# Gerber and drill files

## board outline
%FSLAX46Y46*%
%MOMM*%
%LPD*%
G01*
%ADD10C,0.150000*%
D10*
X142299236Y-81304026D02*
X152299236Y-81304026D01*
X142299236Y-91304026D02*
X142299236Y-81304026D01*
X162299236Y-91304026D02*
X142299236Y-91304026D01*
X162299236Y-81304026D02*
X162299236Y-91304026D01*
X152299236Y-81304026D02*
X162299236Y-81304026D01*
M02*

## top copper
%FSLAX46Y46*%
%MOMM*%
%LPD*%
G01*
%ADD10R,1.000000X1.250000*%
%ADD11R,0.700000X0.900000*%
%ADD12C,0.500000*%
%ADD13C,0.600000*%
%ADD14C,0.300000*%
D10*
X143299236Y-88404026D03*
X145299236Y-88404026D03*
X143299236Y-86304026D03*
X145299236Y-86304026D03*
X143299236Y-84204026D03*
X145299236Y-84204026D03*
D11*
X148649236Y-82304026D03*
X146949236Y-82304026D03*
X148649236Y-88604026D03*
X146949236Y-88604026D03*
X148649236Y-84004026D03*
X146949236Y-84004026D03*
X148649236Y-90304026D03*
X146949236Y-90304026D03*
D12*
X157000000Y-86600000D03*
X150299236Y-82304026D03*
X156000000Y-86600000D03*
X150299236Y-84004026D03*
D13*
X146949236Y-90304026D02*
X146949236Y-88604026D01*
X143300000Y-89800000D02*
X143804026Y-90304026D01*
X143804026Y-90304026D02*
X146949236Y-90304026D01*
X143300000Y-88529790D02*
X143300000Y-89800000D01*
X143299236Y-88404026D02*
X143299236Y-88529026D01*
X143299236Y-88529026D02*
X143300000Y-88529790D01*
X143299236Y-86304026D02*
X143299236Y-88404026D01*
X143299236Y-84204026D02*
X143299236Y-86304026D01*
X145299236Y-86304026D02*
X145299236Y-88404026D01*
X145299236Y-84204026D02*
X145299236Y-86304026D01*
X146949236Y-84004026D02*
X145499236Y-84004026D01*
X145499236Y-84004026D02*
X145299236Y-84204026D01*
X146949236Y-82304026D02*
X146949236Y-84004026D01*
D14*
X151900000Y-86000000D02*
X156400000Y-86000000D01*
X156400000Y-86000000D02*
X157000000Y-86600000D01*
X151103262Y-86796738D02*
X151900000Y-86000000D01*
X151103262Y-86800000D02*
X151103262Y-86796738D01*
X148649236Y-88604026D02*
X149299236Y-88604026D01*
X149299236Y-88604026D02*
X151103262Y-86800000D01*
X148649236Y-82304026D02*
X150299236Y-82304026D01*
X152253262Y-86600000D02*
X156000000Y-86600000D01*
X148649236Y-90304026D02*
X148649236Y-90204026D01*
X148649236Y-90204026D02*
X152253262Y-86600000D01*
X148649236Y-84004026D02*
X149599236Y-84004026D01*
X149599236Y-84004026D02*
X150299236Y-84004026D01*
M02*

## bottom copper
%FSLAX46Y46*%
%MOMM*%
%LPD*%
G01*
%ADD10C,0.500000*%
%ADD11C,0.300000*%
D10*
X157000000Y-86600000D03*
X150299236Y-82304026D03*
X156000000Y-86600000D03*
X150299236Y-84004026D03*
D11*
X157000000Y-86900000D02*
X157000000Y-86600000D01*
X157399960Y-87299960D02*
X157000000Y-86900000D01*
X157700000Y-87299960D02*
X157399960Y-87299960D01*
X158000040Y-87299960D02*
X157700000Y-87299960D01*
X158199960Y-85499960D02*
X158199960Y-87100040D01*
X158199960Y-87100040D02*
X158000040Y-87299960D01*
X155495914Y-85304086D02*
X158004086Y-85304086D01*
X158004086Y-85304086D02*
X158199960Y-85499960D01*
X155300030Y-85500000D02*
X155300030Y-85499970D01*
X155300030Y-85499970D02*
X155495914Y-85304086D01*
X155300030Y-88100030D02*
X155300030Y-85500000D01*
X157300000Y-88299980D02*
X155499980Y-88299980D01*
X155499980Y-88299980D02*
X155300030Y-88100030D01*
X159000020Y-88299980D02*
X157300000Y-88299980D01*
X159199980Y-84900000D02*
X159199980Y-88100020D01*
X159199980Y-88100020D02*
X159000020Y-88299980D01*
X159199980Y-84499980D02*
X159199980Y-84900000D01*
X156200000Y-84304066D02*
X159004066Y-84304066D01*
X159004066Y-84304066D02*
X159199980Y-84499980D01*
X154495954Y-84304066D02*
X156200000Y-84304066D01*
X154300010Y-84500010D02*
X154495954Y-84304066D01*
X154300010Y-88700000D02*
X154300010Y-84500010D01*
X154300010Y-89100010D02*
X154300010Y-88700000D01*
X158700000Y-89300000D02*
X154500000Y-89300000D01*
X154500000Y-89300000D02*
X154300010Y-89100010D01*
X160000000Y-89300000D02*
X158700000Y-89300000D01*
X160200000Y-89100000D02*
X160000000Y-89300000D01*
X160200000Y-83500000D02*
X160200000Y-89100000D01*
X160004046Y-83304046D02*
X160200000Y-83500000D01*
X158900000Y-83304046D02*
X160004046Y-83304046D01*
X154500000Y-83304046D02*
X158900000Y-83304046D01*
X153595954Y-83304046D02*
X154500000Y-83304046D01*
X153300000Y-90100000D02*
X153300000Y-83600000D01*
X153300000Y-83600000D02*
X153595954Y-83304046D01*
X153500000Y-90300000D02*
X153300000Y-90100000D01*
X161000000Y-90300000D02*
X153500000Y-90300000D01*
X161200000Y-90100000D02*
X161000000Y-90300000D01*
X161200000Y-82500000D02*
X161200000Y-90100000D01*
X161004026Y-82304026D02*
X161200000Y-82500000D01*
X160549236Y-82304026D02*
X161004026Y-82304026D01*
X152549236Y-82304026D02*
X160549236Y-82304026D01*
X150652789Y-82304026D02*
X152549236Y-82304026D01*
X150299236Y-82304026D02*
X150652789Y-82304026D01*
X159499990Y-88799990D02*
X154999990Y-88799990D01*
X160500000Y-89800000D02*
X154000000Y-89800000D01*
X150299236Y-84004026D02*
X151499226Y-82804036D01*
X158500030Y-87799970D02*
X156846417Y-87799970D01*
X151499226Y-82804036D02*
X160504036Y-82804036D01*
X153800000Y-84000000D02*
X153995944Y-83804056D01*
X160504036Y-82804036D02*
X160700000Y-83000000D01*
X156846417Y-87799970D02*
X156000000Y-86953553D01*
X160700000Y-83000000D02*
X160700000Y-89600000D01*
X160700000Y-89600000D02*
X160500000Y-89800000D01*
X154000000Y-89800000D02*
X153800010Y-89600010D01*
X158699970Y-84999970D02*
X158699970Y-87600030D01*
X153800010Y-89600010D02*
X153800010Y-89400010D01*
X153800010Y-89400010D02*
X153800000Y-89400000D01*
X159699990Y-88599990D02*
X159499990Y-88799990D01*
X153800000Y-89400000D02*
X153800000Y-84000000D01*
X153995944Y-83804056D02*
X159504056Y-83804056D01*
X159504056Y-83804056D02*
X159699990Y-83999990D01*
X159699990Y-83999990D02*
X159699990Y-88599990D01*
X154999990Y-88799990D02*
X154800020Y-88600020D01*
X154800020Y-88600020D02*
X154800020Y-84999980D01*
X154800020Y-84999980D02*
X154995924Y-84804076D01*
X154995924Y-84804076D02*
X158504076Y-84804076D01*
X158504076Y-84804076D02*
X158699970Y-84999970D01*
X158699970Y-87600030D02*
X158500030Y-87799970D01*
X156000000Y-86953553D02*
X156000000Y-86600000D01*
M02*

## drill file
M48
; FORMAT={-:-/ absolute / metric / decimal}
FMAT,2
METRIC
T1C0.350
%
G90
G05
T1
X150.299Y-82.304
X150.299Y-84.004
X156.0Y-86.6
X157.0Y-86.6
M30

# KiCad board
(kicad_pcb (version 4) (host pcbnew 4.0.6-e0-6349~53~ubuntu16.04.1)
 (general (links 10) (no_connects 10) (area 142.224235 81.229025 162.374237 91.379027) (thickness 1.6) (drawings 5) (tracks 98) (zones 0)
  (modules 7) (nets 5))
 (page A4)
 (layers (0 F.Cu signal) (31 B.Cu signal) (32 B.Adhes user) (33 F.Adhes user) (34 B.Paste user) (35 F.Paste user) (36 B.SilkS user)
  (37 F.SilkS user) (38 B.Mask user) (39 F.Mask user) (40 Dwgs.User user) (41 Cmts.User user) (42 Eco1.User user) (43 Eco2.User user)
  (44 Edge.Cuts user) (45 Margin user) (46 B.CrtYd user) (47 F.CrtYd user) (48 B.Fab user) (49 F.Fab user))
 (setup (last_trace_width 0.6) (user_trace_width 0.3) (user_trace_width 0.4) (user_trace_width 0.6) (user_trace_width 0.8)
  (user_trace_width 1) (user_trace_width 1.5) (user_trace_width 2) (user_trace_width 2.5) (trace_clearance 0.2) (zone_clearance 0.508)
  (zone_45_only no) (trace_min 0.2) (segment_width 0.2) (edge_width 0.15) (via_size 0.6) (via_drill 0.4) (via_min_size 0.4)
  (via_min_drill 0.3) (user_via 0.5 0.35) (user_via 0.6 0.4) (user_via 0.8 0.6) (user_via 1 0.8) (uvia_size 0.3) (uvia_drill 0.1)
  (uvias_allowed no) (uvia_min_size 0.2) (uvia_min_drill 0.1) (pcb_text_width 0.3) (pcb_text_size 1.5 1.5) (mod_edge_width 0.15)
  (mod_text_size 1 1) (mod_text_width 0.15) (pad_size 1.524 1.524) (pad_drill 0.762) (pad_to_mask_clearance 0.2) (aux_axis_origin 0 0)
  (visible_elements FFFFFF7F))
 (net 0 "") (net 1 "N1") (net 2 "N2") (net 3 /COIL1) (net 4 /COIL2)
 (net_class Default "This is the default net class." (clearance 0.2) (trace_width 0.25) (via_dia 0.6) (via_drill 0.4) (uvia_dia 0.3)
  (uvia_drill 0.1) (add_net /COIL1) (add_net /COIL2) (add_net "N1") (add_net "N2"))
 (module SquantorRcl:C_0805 (layer F.Cu) (at 144.299236 88.404026)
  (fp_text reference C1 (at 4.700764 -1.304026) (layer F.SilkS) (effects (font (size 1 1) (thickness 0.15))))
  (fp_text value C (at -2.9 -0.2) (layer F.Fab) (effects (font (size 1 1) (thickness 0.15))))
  (pad 1 smd rect (at -1 0) (size 1 1.25) (layers F.Cu F.Paste F.Mask) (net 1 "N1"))
  (pad 2 smd rect (at 1 0) (size 1 1.25) (layers F.Cu F.Paste F.Mask) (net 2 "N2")))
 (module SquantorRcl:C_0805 (layer F.Cu) (at 144.299236 86.304026)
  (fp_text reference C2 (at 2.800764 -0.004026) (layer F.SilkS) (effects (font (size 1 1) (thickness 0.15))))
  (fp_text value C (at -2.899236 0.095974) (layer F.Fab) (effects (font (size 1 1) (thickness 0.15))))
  (pad 1 smd rect (at -1 0) (size 1 1.25) (layers F.Cu F.Paste F.Mask) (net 1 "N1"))
  (pad 2 smd rect (at 1 0) (size 1 1.25) (layers F.Cu F.Paste F.Mask) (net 2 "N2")))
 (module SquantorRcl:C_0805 (layer F.Cu) (at 144.299236 84.204026)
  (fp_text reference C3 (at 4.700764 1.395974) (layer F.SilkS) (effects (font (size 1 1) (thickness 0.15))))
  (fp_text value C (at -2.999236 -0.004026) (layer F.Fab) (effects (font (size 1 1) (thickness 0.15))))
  (pad 1 smd rect (at -1 0) (size 1 1.25) (layers F.Cu F.Paste F.Mask) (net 1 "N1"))
  (pad 2 smd rect (at 1 0) (size 1 1.25) (layers F.Cu F.Paste F.Mask) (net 2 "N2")))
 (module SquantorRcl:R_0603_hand (layer F.Cu) (at 147.799236 82.304026 180)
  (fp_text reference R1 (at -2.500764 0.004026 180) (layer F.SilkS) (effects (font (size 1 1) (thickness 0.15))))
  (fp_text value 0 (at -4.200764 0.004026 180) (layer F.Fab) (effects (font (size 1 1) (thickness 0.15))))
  (pad 1 smd rect (at -0.85 0 180) (size 0.7 0.9) (layers F.Cu F.Paste F.Mask) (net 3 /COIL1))
  (pad 2 smd rect (at 0.85 0 180) (size 0.7 0.9) (layers F.Cu F.Paste F.Mask) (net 2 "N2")))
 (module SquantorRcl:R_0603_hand (layer F.Cu) (at 147.799236 88.604026 180)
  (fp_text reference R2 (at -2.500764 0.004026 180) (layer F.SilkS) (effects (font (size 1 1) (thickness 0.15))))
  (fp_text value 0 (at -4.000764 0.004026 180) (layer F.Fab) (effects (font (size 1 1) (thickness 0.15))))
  (pad 1 smd rect (at -0.85 0 180) (size 0.7 0.9) (layers F.Cu F.Paste F.Mask) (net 3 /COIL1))
  (pad 2 smd rect (at 0.85 0 180) (size 0.7 0.9) (layers F.Cu F.Paste F.Mask) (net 1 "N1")))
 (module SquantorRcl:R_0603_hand (layer F.Cu) (at 147.799236 84.004026 180)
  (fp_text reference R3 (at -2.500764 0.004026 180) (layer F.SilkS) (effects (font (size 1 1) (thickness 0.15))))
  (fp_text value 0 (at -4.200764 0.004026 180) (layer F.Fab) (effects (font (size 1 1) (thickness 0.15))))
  (pad 1 smd rect (at -0.85 0 180) (size 0.7 0.9) (layers F.Cu F.Paste F.Mask) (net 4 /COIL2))
  (pad 2 smd rect (at 0.85 0 180) (size 0.7 0.9) (layers F.Cu F.Paste F.Mask) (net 2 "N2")))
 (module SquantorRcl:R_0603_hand (layer F.Cu) (at 147.799236 90.304026 180)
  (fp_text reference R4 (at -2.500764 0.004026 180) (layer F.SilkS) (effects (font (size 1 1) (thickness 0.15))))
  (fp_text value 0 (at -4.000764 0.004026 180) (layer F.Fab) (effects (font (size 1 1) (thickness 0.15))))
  (pad 1 smd rect (at -0.85 0 180) (size 0.7 0.9) (layers F.Cu F.Paste F.Mask) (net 4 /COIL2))
  (pad 2 smd rect (at 0.85 0 180) (size 0.7 0.9) (layers F.Cu F.Paste F.Mask) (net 1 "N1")))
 (gr_line (start 142.299236 81.304026) (end 152.299236 81.304026) (layer Edge.Cuts) (width 0.15))
 (gr_line (start 142.299236 91.304026) (end 142.299236 81.304026) (layer Edge.Cuts) (width 0.15))
 (gr_line (start 162.299236 91.304026) (end 142.299236 91.304026) (layer Edge.Cuts) (width 0.15))
 (gr_line (start 162.299236 81.304026) (end 162.299236 91.304026) (layer Edge.Cuts) (width 0.15))
 (gr_line (start 152.299236 81.304026) (end 162.299236 81.304026) (layer Edge.Cuts) (width 0.15))
 (segment (start 146.949236 90.304026) (end 146.949236 88.604026) (width 0.6) (layer F.Cu) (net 1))
 (segment (start 143.3 89.8) (end 143.804026 90.304026) (width 0.6) (layer F.Cu) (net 1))
 (segment (start 143.804026 90.304026) (end 146.949236 90.304026) (width 0.6) (layer F.Cu) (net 1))
 (segment (start 143.3 88.52979) (end 143.3 89.8) (width 0.6) (layer F.Cu) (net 1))
 (segment (start 143.299236 88.404026) (end 143.299236 88.529026) (width 0.6) (layer F.Cu) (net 1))
 (segment (start 143.299236 88.529026) (end 143.3 88.52979) (width 0.6) (layer F.Cu) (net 1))
 (segment (start 143.299236 86.304026) (end 143.299236 88.404026) (width 0.6) (layer F.Cu) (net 1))
 (segment (start 143.299236 84.204026) (end 143.299236 86.304026) (width 0.6) (layer F.Cu) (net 1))
 (segment (start 145.299236 86.304026) (end 145.299236 88.404026) (width 0.6) (layer F.Cu) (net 2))
 (segment (start 145.299236 84.204026) (end 145.299236 86.304026) (width 0.6) (layer F.Cu) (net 2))
 (segment (start 146.949236 84.004026) (end 145.499236 84.004026) (width 0.6) (layer F.Cu) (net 2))
 (segment (start 145.499236 84.004026) (end 145.299236 84.204026) (width 0.6) (layer F.Cu) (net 2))
 (segment (start 146.949236 82.304026) (end 146.949236 84.004026) (width 0.6) (layer F.Cu) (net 2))
 (segment (start 151.9 86) (end 156.4 86) (width 0.3) (layer F.Cu) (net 3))
 (segment (start 156.4 86) (end 157 86.6) (width 0.3) (layer F.Cu) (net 3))
 (segment (start 151.103262 86.796738) (end 151.9 86) (width 0.3) (layer F.Cu) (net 3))
 (segment (start 151.103262 86.8) (end 151.103262 86.796738) (width 0.3) (layer F.Cu) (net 3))
 (via (at 157 86.6) (size 0.5) (drill 0.35) (layers F.Cu B.Cu) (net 3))
 (segment (start 157 86.9) (end 157 86.6) (width 0.3) (layer B.Cu) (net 3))
 (segment (start 157.39996 87.29996) (end 157 86.9) (width 0.3) (layer B.Cu) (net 3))
 (segment (start 157.7 87.29996) (end 157.39996 87.29996) (width 0.3) (layer B.Cu) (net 3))
 (segment (start 148.649236 88.604026) (end 149.299236 88.604026) (width 0.3) (layer F.Cu) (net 3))
 (segment (start 149.299236 88.604026) (end 151.103262 86.8) (width 0.3) (layer F.Cu) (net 3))
 (segment (start 158.00004 87.29996) (end 157.7 87.29996) (width 0.3) (layer B.Cu) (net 3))
 (segment (start 158.19996 85.49996) (end 158.19996 87.10004) (width 0.3) (layer B.Cu) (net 3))
 (segment (start 158.19996 87.10004) (end 158.00004 87.29996) (width 0.3) (layer B.Cu) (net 3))
 (segment (start 155.495914 85.304086) (end 158.004086 85.304086) (width 0.3) (layer B.Cu) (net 3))
 (segment (start 158.004086 85.304086) (end 158.19996 85.49996) (width 0.3) (layer B.Cu) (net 3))
 (segment (start 155.30003 85.5) (end 155.30003 85.49997) (width 0.3) (layer B.Cu) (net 3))
 (segment (start 155.30003 85.49997) (end 155.495914 85.304086) (width 0.3) (layer B.Cu) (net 3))
 (segment (start 155.30003 88.10003) (end 155.30003 85.5) (width 0.3) (layer B.Cu) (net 3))
 (segment (start 157.3 88.29998) (end 155.49998 88.29998) (width 0.3) (layer B.Cu) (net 3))
 (segment (start 155.49998 88.29998) (end 155.30003 88.10003) (width 0.3) (layer B.Cu) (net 3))
 (segment (start 159.00002 88.29998) (end 157.3 88.29998) (width 0.3) (layer B.Cu) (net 3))
 (segment (start 159.19998 84.9) (end 159.19998 88.10002) (width 0.3) (layer B.Cu) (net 3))
 (segment (start 159.19998 88.10002) (end 159.00002 88.29998) (width 0.3) (layer B.Cu) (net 3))
 (segment (start 159.19998 84.49998) (end 159.19998 84.9) (width 0.3) (layer B.Cu) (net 3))
 (segment (start 156.2 84.304066) (end 159.004066 84.304066) (width 0.3) (layer B.Cu) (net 3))
 (segment (start 159.004066 84.304066) (end 159.19998 84.49998) (width 0.3) (layer B.Cu) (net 3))
 (segment (start 154.495954 84.304066) (end 156.2 84.304066) (width 0.3) (layer B.Cu) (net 3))
 (segment (start 154.30001 84.50001) (end 154.495954 84.304066) (width 0.3) (layer B.Cu) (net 3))
 (segment (start 154.30001 88.7) (end 154.30001 84.50001) (width 0.3) (layer B.Cu) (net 3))
 (segment (start 154.30001 89.10001) (end 154.30001 88.7) (width 0.3) (layer B.Cu) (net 3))
 (segment (start 158.7 89.3) (end 154.5 89.3) (width 0.3) (layer B.Cu) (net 3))
 (segment (start 154.5 89.3) (end 154.30001 89.10001) (width 0.3) (layer B.Cu) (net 3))
 (segment (start 160 89.3) (end 158.7 89.3) (width 0.3) (layer B.Cu) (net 3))
 (segment (start 160.2 89.1) (end 160 89.3) (width 0.3) (layer B.Cu) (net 3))
 (segment (start 160.2 83.5) (end 160.2 89.1) (width 0.3) (layer B.Cu) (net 3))
 (segment (start 160.004046 83.304046) (end 160.2 83.5) (width 0.3) (layer B.Cu) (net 3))
 (segment (start 158.9 83.304046) (end 160.004046 83.304046) (width 0.3) (layer B.Cu) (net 3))
 (segment (start 154.5 83.304046) (end 158.9 83.304046) (width 0.3) (layer B.Cu) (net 3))
 (segment (start 153.595954 83.304046) (end 154.5 83.304046) (width 0.3) (layer B.Cu) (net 3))
 (segment (start 153.3 90.1) (end 153.3 83.6) (width 0.3) (layer B.Cu) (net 3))
 (segment (start 153.3 83.6) (end 153.595954 83.304046) (width 0.3) (layer B.Cu) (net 3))
 (segment (start 153.5 90.3) (end 153.3 90.1) (width 0.3) (layer B.Cu) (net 3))
 (segment (start 161 90.3) (end 153.5 90.3) (width 0.3) (layer B.Cu) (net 3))
 (segment (start 161.2 90.1) (end 161 90.3) (width 0.3) (layer B.Cu) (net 3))
 (segment (start 161.2 82.5) (end 161.2 90.1) (width 0.3) (layer B.Cu) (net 3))
 (segment (start 161.004026 82.304026) (end 161.2 82.5) (width 0.3) (layer B.Cu) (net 3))
 (segment (start 160.549236 82.304026) (end 161.004026 82.304026) (width 0.3) (layer B.Cu) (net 3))
 (segment (start 152.549236 82.304026) (end 160.549236 82.304026) (width 0.3) (layer B.Cu) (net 3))
 (segment (start 150.652789 82.304026) (end 152.549236 82.304026) (width 0.3) (layer B.Cu) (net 3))
 (segment (start 150.299236 82.304026) (end 150.652789 82.304026) (width 0.3) (layer B.Cu) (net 3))
 (segment (start 148.649236 82.304026) (end 150.299236 82.304026) (width 0.3) (layer F.Cu) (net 3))
 (via (at 150.299236 82.304026) (size 0.5) (drill 0.35) (layers F.Cu B.Cu) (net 3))
 (segment (start 159.49999 88.79999) (end 154.99999 88.79999) (width 0.3) (layer B.Cu) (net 4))
 (segment (start 160.5 89.8) (end 154 89.8) (width 0.3) (layer B.Cu) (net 4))
 (segment (start 150.299236 84.004026) (end 151.499226 82.804036) (width 0.3) (layer B.Cu) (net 4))
 (segment (start 158.50003 87.79997) (end 156.846417 87.79997) (width 0.3) (layer B.Cu) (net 4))
 (segment (start 151.499226 82.804036) (end 160.504036 82.804036) (width 0.3) (layer B.Cu) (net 4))
 (segment (start 153.8 84) (end 153.995944 83.804056) (width 0.3) (layer B.Cu) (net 4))
 (segment (start 160.504036 82.804036) (end 160.7 83) (width 0.3) (layer B.Cu) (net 4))
 (segment (start 156.846417 87.79997) (end 156 86.953553) (width 0.3) (layer B.Cu) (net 4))
 (segment (start 160.7 83) (end 160.7 89.6) (width 0.3) (layer B.Cu) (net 4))
 (segment (start 160.7 89.6) (end 160.5 89.8) (width 0.3) (layer B.Cu) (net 4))
 (segment (start 154 89.8) (end 153.80001 89.60001) (width 0.3) (layer B.Cu) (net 4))
 (segment (start 158.69997 84.99997) (end 158.69997 87.60003) (width 0.3) (layer B.Cu) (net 4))
 (segment (start 153.80001 89.60001) (end 153.80001 89.40001) (width 0.3) (layer B.Cu) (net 4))
 (segment (start 153.80001 89.40001) (end 153.8 89.4) (width 0.3) (layer B.Cu) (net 4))
 (segment (start 159.69999 88.59999) (end 159.49999 88.79999) (width 0.3) (layer B.Cu) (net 4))
 (segment (start 153.8 89.4) (end 153.8 84) (width 0.3) (layer B.Cu) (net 4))
 (segment (start 153.995944 83.804056) (end 159.504056 83.804056) (width 0.3) (layer B.Cu) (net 4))
 (segment (start 159.504056 83.804056) (end 159.69999 83.99999) (width 0.3) (layer B.Cu) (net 4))
 (segment (start 159.69999 83.99999) (end 159.69999 88.59999) (width 0.3) (layer B.Cu) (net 4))
 (segment (start 154.99999 88.79999) (end 154.80002 88.60002) (width 0.3) (layer B.Cu) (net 4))
 (segment (start 154.80002 88.60002) (end 154.80002 84.99998) (width 0.3) (layer B.Cu) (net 4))
 (segment (start 154.80002 84.99998) (end 154.995924 84.804076) (width 0.3) (layer B.Cu) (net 4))
 (segment (start 154.995924 84.804076) (end 158.504076 84.804076) (width 0.3) (layer B.Cu) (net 4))
 (segment (start 158.504076 84.804076) (end 158.69997 84.99997) (width 0.3) (layer B.Cu) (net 4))
 (segment (start 158.69997 87.60003) (end 158.50003 87.79997) (width 0.3) (layer B.Cu) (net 4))
 (segment (start 156 86.953553) (end 156 86.6) (width 0.3) (layer B.Cu) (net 4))
 (segment (start 152.253262 86.6) (end 156 86.6) (width 0.3) (layer F.Cu) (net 4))
 (segment (start 148.649236 90.304026) (end 148.649236 90.204026) (width 0.3) (layer F.Cu) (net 4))
 (segment (start 148.649236 90.204026) (end 152.253262 86.6) (width 0.3) (layer F.Cu) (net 4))
 (via (at 156 86.6) (size 0.5) (drill 0.35) (layers F.Cu B.Cu) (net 4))
 (segment (start 148.649236 84.004026) (end 149.599236 84.004026) (width 0.3) (layer F.Cu) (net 4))
 (via (at 150.299236 84.004026) (size 0.5) (drill 0.35) (layers F.Cu B.Cu) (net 4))
 (segment (start 149.599236 84.004026) (end 150.299236 84.004026) (width 0.3) (layer F.Cu) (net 4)))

